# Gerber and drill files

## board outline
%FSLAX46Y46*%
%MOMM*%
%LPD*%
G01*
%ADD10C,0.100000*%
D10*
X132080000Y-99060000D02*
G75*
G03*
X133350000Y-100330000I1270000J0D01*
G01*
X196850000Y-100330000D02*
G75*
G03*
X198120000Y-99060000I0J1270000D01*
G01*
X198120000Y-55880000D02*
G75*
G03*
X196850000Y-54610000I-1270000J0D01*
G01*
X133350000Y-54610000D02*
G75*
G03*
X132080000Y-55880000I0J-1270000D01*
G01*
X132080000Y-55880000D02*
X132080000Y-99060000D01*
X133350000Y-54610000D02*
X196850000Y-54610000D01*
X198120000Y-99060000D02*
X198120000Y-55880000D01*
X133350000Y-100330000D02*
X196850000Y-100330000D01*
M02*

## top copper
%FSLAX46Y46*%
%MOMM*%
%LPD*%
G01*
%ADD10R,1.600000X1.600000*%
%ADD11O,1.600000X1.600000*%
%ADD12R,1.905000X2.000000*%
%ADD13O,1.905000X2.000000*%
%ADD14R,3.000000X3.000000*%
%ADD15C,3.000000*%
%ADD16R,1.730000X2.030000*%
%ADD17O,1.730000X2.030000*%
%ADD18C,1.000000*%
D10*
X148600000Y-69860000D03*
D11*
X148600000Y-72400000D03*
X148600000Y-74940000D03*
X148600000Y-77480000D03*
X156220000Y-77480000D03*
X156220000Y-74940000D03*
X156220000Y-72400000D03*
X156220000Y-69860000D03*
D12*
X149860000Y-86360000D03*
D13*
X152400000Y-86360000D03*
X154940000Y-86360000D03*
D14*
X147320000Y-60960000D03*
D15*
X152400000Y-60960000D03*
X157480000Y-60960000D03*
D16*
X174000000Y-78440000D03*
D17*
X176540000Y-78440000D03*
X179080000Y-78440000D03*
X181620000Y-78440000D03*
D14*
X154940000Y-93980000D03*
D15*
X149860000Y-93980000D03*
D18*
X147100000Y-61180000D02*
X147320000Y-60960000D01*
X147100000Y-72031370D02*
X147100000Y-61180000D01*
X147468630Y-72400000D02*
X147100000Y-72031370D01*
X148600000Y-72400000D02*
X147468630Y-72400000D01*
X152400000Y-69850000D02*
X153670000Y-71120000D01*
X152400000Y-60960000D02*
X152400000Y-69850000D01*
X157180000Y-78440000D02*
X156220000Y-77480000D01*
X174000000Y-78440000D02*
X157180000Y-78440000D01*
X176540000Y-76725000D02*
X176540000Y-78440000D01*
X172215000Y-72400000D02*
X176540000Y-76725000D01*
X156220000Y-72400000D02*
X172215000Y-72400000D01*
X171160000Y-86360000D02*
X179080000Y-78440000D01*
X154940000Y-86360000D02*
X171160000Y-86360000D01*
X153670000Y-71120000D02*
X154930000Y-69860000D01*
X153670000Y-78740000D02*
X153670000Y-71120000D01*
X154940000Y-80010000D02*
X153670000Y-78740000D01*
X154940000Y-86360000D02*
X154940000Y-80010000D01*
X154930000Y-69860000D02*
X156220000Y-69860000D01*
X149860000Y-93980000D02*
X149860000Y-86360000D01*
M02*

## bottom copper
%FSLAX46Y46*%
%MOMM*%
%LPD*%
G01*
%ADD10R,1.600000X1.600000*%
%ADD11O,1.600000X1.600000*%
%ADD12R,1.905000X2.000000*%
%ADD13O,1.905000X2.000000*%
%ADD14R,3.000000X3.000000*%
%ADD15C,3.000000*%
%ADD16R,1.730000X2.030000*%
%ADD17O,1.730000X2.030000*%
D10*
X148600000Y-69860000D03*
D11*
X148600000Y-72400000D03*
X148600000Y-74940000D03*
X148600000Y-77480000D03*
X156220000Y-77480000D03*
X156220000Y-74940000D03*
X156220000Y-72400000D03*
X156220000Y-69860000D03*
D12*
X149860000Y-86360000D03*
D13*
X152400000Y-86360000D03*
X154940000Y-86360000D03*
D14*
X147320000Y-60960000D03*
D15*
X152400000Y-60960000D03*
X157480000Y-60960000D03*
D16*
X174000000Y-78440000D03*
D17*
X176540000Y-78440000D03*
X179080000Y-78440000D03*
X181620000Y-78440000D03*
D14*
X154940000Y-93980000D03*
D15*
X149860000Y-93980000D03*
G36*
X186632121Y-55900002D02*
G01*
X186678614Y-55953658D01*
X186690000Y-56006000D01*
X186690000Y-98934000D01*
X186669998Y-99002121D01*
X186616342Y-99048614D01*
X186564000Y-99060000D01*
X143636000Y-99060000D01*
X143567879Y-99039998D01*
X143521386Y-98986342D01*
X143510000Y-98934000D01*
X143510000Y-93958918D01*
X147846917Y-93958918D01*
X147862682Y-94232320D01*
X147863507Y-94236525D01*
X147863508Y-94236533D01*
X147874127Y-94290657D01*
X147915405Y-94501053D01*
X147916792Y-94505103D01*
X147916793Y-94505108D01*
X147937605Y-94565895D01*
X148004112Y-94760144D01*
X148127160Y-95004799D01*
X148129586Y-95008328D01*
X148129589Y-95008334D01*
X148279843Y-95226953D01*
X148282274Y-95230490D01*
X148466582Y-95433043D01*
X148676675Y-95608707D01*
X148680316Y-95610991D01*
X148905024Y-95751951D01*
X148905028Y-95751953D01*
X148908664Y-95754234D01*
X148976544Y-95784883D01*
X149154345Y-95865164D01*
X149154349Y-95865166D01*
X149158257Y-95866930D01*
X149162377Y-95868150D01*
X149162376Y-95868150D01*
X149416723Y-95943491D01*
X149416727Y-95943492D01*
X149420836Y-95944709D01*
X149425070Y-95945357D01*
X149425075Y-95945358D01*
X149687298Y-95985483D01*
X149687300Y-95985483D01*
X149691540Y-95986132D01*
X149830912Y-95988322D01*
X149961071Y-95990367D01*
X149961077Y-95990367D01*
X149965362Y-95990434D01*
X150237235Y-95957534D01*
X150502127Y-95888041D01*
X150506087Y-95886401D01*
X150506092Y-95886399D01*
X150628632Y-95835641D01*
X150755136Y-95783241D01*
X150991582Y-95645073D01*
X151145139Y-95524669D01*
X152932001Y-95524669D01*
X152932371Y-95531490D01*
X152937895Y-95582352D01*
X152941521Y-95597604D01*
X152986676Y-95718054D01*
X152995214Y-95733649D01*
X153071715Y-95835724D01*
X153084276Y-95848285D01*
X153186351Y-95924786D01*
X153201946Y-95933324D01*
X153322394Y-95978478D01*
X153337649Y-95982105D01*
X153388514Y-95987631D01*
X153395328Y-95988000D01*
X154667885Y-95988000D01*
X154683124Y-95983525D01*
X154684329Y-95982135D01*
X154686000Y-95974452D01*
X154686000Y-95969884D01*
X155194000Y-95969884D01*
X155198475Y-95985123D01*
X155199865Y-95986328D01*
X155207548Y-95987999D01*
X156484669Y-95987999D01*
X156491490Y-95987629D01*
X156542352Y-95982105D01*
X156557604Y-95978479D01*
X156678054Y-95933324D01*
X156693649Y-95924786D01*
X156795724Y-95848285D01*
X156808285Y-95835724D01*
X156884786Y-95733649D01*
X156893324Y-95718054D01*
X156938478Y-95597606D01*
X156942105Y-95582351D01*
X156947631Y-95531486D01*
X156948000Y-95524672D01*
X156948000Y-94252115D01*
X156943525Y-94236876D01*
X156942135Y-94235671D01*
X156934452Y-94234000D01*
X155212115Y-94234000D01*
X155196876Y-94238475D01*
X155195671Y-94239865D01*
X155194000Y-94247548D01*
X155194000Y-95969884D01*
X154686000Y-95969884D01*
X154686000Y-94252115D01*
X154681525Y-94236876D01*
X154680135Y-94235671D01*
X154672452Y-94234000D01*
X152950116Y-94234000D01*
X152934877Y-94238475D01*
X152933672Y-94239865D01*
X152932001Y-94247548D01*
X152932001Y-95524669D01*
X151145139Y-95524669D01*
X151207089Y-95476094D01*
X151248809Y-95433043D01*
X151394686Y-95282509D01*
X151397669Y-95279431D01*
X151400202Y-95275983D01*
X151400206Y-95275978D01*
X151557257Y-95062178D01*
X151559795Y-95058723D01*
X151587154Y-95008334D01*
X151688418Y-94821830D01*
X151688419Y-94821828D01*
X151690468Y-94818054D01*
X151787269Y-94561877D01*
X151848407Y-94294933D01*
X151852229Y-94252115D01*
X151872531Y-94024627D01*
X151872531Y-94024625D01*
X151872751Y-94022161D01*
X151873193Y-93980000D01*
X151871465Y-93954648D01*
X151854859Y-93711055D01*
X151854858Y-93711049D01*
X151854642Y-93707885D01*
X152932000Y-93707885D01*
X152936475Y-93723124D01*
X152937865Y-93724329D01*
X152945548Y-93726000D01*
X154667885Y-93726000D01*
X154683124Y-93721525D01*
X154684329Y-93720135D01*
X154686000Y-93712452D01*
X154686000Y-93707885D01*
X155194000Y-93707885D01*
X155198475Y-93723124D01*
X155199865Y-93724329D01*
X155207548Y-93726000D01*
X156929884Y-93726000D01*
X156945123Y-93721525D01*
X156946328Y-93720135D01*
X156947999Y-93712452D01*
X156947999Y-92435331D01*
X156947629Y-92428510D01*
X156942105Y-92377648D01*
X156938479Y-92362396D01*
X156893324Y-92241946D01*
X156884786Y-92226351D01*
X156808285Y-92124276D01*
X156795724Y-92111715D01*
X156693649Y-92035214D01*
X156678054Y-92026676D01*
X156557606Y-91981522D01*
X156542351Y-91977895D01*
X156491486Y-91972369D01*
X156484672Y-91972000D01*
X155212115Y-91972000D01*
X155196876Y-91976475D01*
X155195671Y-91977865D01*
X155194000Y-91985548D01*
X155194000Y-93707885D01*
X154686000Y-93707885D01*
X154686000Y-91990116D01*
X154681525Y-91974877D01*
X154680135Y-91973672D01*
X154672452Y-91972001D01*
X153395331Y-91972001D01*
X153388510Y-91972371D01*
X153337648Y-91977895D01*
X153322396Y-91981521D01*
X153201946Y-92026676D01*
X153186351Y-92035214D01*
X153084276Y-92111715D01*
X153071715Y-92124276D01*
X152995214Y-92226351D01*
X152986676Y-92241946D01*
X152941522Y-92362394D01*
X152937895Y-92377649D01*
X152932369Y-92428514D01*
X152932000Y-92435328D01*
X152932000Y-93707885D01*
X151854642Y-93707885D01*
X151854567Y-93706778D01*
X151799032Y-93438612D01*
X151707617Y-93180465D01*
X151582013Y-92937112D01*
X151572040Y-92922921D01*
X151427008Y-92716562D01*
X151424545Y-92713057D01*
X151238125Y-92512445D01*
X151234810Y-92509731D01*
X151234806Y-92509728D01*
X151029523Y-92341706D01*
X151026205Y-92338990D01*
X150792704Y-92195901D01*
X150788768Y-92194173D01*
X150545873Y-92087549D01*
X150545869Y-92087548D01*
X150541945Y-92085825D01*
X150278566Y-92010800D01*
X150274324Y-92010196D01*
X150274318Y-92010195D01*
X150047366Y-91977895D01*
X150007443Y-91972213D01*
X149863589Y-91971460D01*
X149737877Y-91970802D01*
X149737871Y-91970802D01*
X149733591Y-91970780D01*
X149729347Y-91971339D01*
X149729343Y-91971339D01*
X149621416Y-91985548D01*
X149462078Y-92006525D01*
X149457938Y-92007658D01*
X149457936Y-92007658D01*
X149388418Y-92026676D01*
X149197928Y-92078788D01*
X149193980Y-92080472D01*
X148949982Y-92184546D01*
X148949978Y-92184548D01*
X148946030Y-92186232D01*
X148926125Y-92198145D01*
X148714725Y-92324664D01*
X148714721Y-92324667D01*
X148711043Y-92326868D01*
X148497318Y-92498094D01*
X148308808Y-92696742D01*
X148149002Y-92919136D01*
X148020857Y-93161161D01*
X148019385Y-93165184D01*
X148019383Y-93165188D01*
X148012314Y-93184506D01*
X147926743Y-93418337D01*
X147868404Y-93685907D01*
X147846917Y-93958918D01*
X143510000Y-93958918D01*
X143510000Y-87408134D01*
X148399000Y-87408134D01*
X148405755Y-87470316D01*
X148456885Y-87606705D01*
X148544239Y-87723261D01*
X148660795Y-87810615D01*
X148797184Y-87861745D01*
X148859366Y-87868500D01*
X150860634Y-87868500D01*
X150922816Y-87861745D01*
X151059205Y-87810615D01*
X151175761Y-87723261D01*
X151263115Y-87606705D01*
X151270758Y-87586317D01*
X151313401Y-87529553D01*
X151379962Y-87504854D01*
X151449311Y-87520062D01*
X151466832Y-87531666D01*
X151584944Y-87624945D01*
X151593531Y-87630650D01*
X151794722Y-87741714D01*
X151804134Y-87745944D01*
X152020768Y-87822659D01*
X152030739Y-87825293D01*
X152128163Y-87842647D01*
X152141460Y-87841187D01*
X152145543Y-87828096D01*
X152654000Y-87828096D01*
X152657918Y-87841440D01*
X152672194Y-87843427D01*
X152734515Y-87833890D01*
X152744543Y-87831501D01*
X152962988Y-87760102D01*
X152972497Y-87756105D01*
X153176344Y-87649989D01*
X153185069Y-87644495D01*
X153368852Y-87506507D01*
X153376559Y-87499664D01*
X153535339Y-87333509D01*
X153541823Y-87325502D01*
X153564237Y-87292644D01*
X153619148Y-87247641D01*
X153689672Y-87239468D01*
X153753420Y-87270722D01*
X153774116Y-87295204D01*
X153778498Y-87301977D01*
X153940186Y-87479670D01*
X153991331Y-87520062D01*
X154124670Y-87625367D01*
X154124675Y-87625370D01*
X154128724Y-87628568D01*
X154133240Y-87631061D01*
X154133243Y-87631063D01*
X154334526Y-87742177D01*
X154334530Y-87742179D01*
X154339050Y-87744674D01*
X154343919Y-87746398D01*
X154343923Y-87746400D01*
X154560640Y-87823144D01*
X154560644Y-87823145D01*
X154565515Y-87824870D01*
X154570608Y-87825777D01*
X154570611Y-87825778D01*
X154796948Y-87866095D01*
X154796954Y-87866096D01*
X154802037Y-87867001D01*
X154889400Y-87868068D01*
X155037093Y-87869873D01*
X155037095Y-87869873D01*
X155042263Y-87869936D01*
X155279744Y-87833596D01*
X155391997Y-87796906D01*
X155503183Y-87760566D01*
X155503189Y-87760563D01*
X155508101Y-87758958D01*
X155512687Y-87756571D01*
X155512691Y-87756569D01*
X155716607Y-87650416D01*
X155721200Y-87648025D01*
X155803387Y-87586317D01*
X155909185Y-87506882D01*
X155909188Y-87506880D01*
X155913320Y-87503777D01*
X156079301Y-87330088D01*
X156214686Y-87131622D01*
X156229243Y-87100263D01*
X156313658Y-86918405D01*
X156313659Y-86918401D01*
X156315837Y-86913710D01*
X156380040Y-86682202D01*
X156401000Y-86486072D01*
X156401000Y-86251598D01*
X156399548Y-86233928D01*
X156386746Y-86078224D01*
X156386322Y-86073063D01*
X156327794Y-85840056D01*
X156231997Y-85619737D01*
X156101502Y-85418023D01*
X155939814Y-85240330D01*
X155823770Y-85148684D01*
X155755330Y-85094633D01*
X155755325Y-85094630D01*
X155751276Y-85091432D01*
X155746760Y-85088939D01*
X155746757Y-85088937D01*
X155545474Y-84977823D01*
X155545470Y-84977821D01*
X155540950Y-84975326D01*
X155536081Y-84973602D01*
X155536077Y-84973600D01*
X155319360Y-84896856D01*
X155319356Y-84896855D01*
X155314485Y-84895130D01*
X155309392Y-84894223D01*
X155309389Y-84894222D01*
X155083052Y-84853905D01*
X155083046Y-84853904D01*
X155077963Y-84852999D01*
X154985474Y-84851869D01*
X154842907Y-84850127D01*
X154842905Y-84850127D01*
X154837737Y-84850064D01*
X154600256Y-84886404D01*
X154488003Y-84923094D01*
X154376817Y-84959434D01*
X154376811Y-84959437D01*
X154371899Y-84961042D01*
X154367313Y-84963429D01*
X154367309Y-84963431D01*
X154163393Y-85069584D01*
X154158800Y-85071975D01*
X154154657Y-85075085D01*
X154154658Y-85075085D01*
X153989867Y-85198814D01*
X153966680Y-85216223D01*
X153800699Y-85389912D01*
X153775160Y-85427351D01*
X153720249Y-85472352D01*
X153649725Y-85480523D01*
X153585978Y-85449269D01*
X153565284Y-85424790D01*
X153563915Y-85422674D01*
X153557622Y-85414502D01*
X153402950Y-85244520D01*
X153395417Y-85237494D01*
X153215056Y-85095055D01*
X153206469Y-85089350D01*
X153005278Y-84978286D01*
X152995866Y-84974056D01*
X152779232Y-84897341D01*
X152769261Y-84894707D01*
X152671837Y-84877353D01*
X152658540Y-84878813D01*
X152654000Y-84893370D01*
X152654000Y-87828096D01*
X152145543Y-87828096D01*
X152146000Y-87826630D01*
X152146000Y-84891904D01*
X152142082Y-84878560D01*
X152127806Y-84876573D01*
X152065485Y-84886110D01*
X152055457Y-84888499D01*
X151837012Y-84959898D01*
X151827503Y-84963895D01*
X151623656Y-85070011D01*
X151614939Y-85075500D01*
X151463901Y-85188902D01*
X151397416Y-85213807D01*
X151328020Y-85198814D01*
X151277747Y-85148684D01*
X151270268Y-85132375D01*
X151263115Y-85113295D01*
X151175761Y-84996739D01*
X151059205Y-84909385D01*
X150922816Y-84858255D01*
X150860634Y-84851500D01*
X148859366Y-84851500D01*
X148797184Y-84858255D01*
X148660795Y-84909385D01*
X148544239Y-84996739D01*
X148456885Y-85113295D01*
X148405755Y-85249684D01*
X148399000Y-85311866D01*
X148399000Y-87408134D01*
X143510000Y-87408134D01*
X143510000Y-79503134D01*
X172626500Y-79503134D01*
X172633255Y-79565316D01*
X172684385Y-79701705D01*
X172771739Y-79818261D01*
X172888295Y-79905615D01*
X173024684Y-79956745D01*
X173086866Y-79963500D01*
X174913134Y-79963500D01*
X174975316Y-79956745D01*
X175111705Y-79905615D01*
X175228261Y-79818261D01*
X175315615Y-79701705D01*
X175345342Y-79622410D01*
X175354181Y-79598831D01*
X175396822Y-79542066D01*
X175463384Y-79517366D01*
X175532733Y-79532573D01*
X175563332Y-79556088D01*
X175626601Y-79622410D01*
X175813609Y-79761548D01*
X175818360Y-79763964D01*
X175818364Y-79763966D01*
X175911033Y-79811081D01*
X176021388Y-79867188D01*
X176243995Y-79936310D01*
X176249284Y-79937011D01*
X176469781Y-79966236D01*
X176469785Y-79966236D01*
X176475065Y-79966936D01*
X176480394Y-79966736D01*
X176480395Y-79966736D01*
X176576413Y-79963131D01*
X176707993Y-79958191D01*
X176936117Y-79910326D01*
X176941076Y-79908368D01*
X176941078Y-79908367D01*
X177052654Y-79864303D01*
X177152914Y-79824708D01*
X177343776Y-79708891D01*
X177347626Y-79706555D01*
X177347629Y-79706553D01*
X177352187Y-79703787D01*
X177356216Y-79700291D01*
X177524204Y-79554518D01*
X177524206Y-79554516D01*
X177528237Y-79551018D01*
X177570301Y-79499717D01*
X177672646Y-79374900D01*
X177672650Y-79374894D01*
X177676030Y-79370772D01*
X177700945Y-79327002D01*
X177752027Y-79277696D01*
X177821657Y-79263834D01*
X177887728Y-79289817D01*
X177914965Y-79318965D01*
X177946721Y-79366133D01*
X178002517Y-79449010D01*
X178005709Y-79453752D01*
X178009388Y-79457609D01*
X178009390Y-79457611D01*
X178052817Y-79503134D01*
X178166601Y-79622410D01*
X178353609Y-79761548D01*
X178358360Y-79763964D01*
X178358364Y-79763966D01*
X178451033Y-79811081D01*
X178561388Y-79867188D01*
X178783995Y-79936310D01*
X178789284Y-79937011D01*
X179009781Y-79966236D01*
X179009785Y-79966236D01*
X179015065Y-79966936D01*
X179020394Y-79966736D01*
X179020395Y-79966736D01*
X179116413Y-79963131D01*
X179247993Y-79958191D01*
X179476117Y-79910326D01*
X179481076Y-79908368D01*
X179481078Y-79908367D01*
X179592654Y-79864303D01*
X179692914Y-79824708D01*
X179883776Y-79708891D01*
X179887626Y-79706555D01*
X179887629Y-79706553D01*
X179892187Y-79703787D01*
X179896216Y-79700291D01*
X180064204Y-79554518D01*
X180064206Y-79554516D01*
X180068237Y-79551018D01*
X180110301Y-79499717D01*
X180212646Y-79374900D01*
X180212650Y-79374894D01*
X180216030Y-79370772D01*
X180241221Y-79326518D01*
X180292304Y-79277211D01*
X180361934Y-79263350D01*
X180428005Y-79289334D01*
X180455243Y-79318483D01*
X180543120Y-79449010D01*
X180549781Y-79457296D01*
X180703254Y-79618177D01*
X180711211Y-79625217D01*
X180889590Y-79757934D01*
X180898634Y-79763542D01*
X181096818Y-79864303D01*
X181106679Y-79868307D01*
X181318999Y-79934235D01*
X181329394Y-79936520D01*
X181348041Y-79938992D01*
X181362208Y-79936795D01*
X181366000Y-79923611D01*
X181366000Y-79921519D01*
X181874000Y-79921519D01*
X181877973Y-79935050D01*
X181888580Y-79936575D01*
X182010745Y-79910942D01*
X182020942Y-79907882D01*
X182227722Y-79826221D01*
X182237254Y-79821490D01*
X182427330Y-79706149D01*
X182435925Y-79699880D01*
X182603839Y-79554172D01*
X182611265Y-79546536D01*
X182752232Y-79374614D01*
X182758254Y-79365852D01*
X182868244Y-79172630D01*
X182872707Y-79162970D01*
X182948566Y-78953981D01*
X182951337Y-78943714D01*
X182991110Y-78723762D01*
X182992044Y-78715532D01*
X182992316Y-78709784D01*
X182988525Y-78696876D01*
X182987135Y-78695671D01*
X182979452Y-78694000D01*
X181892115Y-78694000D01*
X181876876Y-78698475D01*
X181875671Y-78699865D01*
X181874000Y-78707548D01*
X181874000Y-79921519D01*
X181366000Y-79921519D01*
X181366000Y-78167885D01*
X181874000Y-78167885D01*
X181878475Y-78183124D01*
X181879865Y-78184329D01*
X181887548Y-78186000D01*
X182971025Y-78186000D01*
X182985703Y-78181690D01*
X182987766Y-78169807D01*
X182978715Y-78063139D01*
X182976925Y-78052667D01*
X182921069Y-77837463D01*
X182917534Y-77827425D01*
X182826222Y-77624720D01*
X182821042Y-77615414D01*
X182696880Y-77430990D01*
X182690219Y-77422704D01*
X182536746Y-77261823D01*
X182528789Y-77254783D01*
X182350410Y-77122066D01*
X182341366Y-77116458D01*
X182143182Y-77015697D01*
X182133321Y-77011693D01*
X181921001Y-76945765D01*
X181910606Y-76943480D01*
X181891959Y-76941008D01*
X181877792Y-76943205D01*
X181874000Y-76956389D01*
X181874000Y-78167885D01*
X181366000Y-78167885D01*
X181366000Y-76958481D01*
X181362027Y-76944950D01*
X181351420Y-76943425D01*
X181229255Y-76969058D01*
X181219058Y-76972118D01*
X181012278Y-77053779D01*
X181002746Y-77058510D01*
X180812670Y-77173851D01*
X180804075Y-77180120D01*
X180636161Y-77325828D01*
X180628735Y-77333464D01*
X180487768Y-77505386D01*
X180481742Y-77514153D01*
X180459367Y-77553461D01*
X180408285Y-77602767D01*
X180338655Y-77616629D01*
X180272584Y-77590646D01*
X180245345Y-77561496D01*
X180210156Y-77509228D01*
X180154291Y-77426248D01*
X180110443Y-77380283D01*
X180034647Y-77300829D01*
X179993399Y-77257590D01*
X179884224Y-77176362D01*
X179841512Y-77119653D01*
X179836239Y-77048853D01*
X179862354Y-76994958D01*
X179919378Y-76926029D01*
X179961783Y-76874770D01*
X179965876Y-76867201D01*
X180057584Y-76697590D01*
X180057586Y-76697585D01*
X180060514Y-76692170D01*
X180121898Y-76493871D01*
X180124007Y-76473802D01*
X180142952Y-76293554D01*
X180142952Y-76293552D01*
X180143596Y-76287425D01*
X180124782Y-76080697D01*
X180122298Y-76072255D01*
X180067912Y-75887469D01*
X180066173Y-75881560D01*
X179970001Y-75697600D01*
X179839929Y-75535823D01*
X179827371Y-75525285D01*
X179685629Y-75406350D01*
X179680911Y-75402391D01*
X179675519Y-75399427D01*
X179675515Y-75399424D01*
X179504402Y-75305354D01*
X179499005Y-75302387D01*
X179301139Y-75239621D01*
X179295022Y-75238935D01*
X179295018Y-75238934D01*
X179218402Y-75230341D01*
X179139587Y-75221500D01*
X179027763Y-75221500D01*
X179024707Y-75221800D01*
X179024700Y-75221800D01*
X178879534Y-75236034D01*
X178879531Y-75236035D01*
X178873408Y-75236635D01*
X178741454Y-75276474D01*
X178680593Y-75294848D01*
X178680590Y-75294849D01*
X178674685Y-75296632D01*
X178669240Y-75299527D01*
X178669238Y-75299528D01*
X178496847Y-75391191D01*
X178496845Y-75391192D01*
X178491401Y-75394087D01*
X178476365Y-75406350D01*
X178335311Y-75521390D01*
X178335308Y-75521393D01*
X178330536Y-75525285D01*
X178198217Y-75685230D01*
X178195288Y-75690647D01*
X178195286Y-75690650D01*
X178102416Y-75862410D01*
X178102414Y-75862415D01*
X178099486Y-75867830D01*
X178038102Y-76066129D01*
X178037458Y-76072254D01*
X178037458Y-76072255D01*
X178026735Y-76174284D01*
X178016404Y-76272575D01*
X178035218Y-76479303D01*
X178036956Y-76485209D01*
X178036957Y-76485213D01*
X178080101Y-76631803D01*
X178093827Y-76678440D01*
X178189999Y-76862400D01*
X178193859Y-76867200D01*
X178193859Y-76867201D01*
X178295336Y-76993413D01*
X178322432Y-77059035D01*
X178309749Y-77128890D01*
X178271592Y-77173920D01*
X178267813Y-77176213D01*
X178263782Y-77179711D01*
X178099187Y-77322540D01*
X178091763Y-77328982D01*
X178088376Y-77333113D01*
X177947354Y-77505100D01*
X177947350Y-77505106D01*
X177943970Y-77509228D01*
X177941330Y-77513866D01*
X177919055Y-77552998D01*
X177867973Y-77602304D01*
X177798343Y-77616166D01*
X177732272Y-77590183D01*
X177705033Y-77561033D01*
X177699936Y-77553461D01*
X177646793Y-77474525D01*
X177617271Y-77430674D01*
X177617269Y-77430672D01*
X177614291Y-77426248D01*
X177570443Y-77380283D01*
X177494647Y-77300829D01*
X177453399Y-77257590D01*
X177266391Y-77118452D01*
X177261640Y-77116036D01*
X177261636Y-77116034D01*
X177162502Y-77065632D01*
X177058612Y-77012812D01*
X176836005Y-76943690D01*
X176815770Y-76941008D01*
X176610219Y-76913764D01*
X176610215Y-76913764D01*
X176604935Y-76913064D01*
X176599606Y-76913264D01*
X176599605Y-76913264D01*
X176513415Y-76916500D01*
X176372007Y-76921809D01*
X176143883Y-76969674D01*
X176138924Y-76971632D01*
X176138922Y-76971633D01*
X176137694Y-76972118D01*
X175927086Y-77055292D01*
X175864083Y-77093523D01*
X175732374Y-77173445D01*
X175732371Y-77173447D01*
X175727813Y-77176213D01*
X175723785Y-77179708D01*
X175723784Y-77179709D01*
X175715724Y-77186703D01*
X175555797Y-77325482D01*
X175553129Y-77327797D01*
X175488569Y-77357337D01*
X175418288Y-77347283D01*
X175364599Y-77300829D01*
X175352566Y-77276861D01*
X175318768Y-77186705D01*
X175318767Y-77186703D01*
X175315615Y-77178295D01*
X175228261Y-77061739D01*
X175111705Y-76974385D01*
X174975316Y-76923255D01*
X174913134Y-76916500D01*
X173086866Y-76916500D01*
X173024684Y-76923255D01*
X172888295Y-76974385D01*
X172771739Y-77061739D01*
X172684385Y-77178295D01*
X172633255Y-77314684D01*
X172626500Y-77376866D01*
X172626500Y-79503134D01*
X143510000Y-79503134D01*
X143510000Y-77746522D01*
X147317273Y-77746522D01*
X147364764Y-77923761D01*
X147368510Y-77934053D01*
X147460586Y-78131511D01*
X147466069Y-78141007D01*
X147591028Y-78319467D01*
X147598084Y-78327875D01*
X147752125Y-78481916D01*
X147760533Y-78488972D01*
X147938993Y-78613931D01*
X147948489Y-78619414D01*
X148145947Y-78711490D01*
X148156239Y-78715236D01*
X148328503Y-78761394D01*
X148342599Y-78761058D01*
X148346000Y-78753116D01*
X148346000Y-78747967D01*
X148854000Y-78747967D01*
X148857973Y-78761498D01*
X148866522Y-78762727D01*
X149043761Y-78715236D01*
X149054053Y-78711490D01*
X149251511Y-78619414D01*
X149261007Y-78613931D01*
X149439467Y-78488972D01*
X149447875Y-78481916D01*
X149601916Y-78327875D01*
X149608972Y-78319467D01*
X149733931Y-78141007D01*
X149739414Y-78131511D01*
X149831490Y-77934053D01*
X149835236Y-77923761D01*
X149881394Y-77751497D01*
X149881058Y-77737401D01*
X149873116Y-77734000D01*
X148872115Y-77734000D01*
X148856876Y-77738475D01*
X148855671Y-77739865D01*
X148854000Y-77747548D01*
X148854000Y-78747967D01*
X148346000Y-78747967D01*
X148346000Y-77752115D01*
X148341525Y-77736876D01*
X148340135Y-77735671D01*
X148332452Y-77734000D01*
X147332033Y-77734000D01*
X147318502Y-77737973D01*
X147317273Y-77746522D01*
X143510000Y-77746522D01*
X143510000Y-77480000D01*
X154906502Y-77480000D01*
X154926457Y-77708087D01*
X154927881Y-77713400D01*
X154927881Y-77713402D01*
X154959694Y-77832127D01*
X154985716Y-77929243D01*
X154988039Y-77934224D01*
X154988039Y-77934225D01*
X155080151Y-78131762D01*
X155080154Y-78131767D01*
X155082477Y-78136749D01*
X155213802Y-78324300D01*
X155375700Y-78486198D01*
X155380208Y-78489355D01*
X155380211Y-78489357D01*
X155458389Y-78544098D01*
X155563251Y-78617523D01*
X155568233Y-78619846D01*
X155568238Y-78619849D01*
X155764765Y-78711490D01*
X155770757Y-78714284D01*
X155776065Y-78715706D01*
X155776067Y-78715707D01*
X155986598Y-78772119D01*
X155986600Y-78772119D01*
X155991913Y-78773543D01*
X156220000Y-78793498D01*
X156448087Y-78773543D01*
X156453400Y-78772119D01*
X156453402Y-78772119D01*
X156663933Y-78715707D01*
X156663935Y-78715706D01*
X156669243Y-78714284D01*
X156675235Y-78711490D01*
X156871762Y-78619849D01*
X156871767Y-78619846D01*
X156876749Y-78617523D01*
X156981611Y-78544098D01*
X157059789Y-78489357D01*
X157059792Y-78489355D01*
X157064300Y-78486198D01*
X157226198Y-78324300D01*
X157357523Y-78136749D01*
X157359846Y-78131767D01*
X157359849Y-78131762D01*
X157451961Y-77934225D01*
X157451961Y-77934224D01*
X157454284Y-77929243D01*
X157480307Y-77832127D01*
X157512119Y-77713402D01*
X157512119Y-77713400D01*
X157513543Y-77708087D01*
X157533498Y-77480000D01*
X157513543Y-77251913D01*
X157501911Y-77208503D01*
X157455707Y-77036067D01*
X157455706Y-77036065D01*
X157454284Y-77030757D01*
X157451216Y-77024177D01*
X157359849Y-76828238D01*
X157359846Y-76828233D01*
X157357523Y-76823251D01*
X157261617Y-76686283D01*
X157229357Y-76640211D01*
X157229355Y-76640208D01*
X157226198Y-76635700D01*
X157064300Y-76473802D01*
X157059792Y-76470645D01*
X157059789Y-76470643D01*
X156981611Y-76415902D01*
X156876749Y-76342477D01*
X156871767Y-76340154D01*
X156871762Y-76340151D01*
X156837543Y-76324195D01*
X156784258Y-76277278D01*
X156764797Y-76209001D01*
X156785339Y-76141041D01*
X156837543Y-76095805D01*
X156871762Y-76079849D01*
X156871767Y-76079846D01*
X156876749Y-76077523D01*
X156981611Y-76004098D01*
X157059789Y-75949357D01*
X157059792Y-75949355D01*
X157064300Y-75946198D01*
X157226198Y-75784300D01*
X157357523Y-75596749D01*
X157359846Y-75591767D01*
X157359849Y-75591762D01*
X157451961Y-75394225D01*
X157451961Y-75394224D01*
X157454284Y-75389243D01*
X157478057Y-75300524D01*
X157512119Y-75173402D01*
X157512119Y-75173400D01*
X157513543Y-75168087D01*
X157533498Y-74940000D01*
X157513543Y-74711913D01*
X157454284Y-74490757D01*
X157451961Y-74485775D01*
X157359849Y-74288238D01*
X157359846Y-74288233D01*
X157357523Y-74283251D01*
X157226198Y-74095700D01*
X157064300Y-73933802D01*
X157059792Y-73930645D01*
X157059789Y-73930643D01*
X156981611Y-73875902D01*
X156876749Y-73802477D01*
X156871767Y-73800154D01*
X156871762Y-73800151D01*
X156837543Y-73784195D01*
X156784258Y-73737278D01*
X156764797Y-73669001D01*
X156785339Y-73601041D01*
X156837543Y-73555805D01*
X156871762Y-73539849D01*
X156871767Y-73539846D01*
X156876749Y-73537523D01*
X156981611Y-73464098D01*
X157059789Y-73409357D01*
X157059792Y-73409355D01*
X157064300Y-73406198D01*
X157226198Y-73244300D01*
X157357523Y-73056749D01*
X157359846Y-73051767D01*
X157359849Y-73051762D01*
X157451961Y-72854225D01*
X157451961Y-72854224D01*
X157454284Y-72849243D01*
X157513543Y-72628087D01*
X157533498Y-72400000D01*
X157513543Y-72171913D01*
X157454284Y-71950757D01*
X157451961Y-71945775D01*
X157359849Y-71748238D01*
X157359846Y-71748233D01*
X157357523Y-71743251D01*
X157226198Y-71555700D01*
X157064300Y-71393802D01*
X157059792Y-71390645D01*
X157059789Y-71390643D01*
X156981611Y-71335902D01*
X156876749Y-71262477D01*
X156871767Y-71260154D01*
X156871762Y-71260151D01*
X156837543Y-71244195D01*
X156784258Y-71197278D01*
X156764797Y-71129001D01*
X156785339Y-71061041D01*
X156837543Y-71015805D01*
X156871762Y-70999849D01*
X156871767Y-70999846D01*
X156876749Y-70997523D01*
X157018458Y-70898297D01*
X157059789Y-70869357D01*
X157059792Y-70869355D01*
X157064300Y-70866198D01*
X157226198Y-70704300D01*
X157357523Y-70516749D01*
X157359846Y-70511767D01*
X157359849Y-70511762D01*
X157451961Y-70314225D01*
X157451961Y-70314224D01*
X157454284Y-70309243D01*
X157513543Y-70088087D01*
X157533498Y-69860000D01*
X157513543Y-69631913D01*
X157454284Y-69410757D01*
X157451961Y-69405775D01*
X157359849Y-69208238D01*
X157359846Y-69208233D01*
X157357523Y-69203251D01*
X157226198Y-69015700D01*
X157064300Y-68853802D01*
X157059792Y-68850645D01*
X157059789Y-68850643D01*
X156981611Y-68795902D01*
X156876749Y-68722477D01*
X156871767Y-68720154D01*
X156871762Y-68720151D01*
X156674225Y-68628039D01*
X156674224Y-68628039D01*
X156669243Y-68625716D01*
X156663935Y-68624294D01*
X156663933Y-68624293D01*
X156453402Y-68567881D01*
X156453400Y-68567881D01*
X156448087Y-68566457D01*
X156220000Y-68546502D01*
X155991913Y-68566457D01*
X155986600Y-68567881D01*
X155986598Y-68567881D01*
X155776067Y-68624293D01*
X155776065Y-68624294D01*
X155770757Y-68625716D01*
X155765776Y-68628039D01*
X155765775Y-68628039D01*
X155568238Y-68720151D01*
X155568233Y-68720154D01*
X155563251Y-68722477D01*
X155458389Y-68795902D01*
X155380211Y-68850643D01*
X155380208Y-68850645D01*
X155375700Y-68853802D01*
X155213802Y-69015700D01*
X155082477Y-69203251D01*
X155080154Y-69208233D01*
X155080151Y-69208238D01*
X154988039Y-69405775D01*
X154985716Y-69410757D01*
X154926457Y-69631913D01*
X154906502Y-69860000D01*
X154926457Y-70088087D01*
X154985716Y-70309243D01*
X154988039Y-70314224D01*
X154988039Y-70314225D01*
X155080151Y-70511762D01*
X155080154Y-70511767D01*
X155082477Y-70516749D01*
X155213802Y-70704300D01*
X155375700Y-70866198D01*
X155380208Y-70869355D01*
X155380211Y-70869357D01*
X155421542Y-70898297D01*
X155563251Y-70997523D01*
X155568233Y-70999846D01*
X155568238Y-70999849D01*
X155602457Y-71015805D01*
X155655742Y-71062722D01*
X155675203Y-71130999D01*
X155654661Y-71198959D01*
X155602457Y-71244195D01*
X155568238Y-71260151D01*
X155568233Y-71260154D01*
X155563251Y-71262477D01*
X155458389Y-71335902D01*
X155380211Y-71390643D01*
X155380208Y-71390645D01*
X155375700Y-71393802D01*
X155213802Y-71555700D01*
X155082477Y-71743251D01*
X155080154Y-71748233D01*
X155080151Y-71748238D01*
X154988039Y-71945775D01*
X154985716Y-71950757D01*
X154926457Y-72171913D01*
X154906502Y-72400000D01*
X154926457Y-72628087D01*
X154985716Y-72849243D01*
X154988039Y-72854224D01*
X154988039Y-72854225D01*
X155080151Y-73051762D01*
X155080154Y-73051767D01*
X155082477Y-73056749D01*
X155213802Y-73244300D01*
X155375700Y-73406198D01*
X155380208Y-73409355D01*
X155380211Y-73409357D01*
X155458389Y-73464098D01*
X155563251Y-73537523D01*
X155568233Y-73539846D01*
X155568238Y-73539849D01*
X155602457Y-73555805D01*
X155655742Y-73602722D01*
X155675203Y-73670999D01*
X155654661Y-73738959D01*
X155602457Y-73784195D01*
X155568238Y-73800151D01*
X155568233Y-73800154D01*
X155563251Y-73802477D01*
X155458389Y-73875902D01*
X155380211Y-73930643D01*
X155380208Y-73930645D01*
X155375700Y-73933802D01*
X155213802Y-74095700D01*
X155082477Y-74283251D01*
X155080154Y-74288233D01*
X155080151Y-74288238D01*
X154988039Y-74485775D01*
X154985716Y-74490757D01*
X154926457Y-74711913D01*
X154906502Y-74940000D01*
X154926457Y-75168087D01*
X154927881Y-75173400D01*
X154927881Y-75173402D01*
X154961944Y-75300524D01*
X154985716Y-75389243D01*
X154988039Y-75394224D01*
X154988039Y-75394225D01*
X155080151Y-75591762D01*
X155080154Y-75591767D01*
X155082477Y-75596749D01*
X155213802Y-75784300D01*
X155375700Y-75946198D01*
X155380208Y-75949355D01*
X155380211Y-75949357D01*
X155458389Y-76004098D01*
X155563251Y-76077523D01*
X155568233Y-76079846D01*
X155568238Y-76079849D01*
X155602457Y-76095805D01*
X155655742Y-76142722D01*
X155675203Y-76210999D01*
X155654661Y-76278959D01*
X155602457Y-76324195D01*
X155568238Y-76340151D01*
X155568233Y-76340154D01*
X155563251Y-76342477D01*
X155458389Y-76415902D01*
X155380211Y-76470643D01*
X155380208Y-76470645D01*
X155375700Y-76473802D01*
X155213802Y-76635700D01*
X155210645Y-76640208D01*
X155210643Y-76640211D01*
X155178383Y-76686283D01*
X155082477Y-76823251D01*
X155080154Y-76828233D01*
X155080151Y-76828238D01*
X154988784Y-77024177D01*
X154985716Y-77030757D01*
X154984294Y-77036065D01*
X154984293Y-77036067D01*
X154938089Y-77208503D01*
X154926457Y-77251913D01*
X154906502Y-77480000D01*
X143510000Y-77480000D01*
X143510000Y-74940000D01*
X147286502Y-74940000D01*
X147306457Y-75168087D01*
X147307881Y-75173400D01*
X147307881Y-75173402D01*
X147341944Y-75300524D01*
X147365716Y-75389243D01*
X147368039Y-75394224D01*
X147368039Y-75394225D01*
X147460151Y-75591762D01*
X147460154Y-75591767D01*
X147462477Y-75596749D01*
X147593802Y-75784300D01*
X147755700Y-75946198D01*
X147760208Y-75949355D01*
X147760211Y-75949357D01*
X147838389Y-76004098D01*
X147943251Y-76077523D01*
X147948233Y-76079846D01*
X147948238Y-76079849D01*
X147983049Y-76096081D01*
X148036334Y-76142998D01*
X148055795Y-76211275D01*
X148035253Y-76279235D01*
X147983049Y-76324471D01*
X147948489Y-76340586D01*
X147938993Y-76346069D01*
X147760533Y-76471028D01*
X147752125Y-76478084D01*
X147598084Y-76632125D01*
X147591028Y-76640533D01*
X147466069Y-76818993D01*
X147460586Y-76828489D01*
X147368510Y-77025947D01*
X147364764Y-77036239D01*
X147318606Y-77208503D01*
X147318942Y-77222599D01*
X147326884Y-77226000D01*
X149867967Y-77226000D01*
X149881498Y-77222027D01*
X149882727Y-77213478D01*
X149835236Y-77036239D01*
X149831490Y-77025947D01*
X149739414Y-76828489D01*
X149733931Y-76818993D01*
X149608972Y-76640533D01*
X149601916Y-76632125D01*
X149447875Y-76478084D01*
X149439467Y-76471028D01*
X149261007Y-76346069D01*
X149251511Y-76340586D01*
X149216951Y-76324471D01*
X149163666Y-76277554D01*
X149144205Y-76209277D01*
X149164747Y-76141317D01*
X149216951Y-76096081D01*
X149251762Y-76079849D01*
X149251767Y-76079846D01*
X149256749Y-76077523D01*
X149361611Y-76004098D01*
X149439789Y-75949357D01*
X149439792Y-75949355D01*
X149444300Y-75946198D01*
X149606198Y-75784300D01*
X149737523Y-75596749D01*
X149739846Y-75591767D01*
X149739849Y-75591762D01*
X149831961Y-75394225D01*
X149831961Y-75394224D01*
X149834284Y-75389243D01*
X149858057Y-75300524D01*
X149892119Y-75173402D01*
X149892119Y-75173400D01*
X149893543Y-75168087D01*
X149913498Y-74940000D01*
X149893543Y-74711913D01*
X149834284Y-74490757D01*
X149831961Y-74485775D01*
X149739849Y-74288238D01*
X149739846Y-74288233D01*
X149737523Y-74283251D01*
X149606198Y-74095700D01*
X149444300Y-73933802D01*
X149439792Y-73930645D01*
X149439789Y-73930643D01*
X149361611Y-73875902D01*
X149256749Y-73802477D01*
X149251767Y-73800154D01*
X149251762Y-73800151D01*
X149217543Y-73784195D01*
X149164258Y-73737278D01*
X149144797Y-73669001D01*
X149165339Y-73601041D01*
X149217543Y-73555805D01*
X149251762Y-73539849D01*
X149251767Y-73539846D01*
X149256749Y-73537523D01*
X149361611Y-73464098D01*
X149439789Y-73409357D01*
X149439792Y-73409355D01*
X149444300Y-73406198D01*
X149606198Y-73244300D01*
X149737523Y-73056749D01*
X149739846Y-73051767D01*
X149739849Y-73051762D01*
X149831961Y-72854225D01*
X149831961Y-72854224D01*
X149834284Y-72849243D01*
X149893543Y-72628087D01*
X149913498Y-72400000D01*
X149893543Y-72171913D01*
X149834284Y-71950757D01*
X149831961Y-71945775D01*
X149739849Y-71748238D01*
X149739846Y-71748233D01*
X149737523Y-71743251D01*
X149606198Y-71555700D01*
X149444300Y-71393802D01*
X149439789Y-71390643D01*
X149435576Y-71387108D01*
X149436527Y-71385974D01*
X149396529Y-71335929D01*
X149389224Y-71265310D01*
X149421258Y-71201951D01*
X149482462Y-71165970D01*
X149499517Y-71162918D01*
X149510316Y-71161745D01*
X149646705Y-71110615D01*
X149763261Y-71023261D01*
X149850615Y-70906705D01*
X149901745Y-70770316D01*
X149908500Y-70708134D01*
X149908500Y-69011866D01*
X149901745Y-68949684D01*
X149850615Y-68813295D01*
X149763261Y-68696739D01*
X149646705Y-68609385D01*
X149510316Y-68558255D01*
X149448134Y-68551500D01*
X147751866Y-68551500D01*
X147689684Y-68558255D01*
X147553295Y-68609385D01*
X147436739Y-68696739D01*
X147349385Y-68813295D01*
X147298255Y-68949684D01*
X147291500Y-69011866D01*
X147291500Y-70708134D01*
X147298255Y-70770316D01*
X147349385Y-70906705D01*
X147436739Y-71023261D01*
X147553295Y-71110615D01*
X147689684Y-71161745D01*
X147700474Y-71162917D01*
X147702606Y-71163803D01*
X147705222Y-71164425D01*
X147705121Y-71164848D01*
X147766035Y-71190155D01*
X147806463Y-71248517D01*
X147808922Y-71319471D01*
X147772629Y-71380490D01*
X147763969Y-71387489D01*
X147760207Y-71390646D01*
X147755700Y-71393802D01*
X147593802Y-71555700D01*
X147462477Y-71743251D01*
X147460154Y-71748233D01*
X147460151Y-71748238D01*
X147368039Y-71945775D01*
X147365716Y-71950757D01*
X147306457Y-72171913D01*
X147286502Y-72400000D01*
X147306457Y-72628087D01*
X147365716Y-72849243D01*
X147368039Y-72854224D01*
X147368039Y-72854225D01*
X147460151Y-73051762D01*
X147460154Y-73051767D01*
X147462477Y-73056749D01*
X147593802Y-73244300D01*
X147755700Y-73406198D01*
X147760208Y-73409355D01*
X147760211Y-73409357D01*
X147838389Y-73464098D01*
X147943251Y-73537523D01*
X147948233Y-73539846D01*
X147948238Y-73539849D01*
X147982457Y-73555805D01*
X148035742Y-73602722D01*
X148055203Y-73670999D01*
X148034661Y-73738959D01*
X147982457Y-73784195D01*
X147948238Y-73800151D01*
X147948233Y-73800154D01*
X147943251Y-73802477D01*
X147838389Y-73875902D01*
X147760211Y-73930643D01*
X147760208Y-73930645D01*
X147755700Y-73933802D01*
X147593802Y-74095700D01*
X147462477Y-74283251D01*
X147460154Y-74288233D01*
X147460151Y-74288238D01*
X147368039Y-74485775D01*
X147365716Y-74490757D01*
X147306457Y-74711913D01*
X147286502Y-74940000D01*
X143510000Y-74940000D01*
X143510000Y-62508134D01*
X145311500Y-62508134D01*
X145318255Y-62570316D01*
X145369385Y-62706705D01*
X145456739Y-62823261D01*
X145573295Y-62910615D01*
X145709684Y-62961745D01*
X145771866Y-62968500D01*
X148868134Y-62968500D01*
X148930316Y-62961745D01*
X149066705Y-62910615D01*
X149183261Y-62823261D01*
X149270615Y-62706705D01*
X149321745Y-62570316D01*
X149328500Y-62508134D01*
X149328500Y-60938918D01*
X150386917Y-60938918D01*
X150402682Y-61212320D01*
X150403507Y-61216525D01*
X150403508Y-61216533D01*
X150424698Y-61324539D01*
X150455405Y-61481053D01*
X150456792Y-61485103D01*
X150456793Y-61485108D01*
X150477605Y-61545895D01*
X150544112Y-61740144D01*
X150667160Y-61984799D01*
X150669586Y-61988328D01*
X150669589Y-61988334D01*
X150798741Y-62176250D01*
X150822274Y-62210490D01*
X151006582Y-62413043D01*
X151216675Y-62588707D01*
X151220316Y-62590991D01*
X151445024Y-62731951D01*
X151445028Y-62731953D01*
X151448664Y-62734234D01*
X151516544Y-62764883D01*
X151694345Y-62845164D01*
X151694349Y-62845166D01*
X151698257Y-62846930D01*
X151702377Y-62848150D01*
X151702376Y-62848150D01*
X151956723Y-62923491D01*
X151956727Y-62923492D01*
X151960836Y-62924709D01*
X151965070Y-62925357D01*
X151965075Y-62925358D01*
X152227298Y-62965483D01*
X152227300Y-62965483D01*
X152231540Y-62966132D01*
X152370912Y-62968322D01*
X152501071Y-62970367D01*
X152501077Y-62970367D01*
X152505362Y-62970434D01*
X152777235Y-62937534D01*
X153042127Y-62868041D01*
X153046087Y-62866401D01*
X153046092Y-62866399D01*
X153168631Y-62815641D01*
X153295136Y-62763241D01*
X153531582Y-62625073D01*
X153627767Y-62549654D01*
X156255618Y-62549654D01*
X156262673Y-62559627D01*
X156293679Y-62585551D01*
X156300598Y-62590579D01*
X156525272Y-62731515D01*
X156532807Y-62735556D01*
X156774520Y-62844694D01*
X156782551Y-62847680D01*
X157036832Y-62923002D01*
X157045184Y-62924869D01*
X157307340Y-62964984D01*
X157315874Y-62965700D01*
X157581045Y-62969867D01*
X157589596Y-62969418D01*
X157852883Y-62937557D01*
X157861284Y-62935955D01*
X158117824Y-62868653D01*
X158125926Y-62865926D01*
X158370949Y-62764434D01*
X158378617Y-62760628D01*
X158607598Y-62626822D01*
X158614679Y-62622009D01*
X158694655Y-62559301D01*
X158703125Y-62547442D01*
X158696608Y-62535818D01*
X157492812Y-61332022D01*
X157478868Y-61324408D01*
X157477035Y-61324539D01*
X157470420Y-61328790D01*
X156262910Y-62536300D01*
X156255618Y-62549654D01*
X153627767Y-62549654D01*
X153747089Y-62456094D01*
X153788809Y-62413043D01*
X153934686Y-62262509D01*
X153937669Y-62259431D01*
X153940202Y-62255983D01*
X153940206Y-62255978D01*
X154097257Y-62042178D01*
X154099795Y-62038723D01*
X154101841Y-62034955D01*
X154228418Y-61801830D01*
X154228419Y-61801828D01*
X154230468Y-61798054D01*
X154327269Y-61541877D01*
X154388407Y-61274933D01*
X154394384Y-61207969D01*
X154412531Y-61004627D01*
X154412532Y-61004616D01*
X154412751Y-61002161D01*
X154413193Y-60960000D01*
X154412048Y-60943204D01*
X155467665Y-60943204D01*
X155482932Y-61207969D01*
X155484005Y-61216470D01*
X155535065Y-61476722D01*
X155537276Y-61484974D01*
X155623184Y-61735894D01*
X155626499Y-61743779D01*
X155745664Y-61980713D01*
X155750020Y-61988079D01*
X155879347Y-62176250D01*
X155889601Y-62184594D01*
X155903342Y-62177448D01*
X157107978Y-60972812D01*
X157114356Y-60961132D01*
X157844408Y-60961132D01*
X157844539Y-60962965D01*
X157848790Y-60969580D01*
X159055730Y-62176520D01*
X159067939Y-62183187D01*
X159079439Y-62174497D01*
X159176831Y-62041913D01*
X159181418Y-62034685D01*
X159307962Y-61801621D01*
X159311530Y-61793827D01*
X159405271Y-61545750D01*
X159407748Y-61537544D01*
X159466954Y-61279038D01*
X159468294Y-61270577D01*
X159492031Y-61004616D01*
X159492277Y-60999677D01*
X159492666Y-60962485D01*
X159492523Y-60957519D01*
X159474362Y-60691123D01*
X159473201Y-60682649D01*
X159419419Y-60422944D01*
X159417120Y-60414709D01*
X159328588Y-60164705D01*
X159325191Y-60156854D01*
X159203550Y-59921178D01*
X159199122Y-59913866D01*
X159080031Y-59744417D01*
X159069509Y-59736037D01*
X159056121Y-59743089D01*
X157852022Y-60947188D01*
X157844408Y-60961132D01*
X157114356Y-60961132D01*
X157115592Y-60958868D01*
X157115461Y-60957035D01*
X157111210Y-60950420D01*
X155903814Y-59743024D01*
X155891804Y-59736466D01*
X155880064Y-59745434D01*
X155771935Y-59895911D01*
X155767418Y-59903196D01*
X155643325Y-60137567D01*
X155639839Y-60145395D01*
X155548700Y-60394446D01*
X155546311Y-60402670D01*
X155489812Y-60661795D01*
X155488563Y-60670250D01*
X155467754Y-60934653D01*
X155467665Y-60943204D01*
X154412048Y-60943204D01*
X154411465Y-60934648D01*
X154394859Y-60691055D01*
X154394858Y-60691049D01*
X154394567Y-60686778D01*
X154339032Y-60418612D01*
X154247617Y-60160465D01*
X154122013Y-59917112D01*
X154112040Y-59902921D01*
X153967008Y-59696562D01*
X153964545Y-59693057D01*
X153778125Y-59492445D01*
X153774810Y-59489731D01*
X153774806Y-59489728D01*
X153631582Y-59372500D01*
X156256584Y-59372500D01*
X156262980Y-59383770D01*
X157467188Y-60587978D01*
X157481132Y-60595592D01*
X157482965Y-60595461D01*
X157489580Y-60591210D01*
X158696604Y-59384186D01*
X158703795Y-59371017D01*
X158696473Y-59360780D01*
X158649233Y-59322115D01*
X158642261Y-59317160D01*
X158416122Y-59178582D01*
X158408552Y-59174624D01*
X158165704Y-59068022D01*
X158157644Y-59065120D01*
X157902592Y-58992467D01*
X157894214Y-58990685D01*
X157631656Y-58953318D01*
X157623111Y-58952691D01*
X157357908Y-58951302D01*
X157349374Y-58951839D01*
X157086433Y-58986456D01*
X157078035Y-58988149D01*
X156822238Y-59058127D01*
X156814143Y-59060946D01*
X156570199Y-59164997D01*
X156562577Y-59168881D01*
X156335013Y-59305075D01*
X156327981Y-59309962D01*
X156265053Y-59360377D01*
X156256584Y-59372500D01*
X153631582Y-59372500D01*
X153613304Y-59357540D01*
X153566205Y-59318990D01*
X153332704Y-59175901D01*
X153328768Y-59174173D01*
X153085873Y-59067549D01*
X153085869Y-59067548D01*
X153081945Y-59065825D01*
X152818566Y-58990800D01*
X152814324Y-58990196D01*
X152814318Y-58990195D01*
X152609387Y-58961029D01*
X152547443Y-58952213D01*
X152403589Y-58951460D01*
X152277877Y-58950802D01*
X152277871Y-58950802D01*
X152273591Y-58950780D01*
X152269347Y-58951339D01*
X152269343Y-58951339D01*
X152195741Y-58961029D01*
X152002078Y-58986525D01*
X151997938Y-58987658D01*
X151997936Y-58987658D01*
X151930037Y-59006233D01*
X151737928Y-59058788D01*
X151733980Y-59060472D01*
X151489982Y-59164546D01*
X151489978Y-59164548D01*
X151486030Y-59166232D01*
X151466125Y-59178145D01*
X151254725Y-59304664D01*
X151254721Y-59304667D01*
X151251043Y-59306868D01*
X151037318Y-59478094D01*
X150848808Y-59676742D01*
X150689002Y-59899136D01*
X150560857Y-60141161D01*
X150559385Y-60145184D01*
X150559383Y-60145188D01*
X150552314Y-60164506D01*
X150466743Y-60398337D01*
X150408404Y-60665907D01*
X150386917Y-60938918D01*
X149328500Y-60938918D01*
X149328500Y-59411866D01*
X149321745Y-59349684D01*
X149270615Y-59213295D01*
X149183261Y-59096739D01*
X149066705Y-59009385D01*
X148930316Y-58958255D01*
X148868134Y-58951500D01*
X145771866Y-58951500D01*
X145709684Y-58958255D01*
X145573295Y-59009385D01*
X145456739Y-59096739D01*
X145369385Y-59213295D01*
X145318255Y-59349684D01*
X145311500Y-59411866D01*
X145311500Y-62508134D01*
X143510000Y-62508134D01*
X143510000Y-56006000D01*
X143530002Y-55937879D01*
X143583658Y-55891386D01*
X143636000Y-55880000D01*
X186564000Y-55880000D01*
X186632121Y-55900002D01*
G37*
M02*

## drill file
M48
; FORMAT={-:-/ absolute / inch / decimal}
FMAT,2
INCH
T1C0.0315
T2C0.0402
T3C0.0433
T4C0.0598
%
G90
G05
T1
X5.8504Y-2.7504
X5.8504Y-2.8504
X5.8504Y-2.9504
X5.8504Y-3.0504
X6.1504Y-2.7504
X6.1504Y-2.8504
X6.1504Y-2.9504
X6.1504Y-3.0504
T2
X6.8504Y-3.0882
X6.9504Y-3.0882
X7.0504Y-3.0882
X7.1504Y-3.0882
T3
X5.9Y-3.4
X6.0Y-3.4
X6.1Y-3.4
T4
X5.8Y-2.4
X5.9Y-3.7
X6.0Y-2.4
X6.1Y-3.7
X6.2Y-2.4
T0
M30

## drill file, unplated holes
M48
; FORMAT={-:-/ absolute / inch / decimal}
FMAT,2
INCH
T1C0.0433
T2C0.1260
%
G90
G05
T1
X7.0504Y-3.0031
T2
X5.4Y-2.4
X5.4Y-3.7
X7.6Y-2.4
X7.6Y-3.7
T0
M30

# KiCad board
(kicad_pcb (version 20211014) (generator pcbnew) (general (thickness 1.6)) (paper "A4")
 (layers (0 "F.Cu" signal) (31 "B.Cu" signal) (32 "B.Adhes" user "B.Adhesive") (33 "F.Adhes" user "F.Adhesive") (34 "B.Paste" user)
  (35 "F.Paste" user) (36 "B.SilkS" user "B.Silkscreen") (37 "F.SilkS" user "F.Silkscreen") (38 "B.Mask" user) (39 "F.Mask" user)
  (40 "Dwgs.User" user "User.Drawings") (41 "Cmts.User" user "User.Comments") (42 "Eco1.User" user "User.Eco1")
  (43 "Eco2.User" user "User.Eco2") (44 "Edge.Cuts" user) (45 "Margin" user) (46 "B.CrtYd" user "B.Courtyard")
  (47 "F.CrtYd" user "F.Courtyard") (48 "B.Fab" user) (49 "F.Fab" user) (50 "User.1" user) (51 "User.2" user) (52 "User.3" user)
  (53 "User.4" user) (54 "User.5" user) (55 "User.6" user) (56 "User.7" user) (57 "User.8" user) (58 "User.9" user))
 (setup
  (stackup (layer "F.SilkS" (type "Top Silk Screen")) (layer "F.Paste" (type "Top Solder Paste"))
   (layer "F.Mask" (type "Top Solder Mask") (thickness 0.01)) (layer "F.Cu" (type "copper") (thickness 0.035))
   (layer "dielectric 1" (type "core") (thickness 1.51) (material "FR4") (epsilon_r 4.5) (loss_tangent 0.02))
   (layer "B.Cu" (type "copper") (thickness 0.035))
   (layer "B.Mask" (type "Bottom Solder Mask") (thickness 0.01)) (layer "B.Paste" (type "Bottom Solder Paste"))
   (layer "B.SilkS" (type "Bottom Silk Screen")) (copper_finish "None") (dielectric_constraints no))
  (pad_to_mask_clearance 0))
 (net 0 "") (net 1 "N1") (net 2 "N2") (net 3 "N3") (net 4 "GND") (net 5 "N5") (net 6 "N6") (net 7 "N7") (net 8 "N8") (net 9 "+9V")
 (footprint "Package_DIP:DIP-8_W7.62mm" (layer "F.Cu") (at 148.6 69.86)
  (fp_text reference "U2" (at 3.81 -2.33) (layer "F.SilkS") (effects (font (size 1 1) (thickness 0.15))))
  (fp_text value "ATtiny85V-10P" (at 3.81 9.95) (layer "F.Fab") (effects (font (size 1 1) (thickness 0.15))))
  (pad "1" thru_hole rect (at 0 0) (size 1.6 1.6) (drill 0.8) (layers *.Cu *.Mask) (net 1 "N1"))
  (pad "2" thru_hole oval (at 0 2.54) (size 1.6 1.6) (drill 0.8) (layers *.Cu *.Mask) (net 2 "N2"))
  (pad "3" thru_hole oval (at 0 5.08) (size 1.6 1.6) (drill 0.8) (layers *.Cu *.Mask) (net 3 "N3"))
  (pad "4" thru_hole oval (at 0 7.62) (size 1.6 1.6) (drill 0.8) (layers *.Cu *.Mask) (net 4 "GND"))
  (pad "5" thru_hole oval (at 7.62 7.62) (size 1.6 1.6) (drill 0.8) (layers *.Cu *.Mask) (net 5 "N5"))
  (pad "6" thru_hole oval (at 7.62 5.08) (size 1.6 1.6) (drill 0.8) (layers *.Cu *.Mask) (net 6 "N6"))
  (pad "7" thru_hole oval (at 7.62 2.54) (size 1.6 1.6) (drill 0.8) (layers *.Cu *.Mask) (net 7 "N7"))
  (pad "8" thru_hole oval (at 7.62 0) (size 1.6 1.6) (drill 0.8) (layers *.Cu *.Mask) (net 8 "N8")))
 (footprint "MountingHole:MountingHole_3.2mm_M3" (layer "F.Cu") (at 137.16 93.98)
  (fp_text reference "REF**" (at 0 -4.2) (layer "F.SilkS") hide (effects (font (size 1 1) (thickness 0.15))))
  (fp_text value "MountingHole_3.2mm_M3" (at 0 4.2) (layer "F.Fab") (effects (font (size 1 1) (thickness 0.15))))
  (pad "" np_thru_hole circle (at 0 0) (size 3.2 3.2) (drill 3.2) (layers *.Cu *.Mask)))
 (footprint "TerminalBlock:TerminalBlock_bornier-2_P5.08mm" (layer "F.Cu") (at 154.94 93.98 180)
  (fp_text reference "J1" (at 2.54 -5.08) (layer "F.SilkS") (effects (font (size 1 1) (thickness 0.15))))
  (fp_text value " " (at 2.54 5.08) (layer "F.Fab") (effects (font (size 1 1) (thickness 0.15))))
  (pad "1" thru_hole rect (at 0 0 180) (size 3 3) (drill 1.52) (layers *.Cu *.Mask) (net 4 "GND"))
  (pad "2" thru_hole circle (at 5.08 0 180) (size 3 3) (drill 1.52) (layers *.Cu *.Mask) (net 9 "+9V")))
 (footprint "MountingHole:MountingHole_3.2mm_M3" (layer "F.Cu") (at 193.04 93.98)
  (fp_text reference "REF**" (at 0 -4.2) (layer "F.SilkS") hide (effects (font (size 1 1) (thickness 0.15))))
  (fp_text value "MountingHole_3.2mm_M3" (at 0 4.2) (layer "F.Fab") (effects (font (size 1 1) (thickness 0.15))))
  (pad "" np_thru_hole circle (at 0 0) (size 3.2 3.2) (drill 3.2) (layers F&B.Cu *.Mask)))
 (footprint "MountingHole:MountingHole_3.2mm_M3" (layer "F.Cu") (at 137.16 60.96)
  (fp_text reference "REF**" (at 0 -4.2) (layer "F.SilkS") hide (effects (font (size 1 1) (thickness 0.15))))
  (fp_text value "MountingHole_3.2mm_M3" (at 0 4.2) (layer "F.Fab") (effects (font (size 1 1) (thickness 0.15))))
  (pad "" np_thru_hole circle (at 0 0) (size 3.2 3.2) (drill 3.2) (layers F&B.Cu *.Mask)))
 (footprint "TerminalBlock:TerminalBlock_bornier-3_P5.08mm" (layer "F.Cu") (at 147.32 60.96)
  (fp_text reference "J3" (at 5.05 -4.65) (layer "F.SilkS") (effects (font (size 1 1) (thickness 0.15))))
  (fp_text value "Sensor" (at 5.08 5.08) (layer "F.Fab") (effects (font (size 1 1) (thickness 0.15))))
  (pad "1" thru_hole rect (at 0 0) (size 3 3) (drill 1.52) (layers *.Cu *.Mask) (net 2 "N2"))
  (pad "2" thru_hole circle (at 5.08 0) (size 3 3) (drill 1.52) (layers *.Cu *.Mask) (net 8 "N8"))
  (pad "3" thru_hole circle (at 10.16 0) (size 3 3) (drill 1.52) (layers *.Cu *.Mask) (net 4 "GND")))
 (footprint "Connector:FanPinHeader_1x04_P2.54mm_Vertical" (layer "F.Cu") (at 174 78.44)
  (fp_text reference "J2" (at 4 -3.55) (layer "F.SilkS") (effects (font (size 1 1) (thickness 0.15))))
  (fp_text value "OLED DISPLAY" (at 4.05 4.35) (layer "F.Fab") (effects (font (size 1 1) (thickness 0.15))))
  (pad "" np_thru_hole circle (at 5.08 -2.16 90) (size 1.1 1.1) (drill 1.1) (layers *.Cu *.Mask))
  (pad "1" thru_hole rect (at 0 0 90) (size 2.03 1.73) (drill 1.02) (layers *.Cu *.Mask) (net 5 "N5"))
  (pad "2" thru_hole oval (at 2.54 0 90) (size 2.03 1.73) (drill 1.02) (layers *.Cu *.Mask) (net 7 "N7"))
  (pad "3" thru_hole oval (at 5.08 0 90) (size 2.03 1.73) (drill 1.02) (layers *.Cu *.Mask) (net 8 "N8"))
  (pad "4" thru_hole oval (at 7.62 0 90) (size 2.03 1.73) (drill 1.02) (layers *.Cu *.Mask) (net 4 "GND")))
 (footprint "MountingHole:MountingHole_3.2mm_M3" (layer "F.Cu") (at 193.04 60.96)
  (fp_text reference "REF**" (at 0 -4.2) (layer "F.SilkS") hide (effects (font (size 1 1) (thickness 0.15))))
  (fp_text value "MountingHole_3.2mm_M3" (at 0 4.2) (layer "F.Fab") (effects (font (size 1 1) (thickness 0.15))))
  (pad "" np_thru_hole circle (at 0 0) (size 3.2 3.2) (drill 3.2) (layers F&B.Cu *.Mask)))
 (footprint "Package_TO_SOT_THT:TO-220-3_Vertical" (layer "F.Cu") (at 149.86 86.36)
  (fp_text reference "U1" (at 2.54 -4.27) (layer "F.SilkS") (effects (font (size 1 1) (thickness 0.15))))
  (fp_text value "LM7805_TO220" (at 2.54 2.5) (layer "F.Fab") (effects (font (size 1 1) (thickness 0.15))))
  (pad "1" thru_hole rect (at 0 0) (size 1.905 2) (drill 1.1) (layers *.Cu *.Mask) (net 9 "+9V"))
  (pad "2" thru_hole oval (at 2.54 0) (size 1.905 2) (drill 1.1) (layers *.Cu *.Mask) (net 4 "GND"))
  (pad "3" thru_hole oval (at 5.08 0) (size 1.905 2) (drill 1.1) (layers *.Cu *.Mask) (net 8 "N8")))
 (gr_line (start 132.08 55.88) (end 132.08 99.06) (layer "Edge.Cuts") (width 0.1))
 (gr_arc (start 133.35 100.33) (mid 132.451974 99.958026) (end 132.08 99.06) (layer "Edge.Cuts") (width 0.1))
 (gr_line (start 133.35 54.61) (end 196.85 54.61) (layer "Edge.Cuts") (width 0.1))
 (gr_line (start 133.35 100.33) (end 196.85 100.33) (layer "Edge.Cuts") (width 0.1))
 (gr_arc (start 132.08 55.88) (mid 132.451974 54.981974) (end 133.35 54.61) (layer "Edge.Cuts") (width 0.1))
 (gr_arc (start 198.12 99.06) (mid 197.748026 99.958026) (end 196.85 100.33) (layer "Edge.Cuts") (width 0.1))
 (gr_arc (start 196.85 54.61) (mid 197.748026 54.981974) (end 198.12 55.88) (layer "Edge.Cuts") (width 0.1))
 (gr_line (start 198.12 99.06) (end 198.12 55.88) (layer "Edge.Cuts") (width 0.1))
 (segment (start 149.86 93.98) (end 149.86 86.36) (width 1) (layer "F.Cu") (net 9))
 (segment (start 157.18 78.44) (end 156.22 77.48) (width 1) (layer "F.Cu") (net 5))
 (segment (start 174 78.44) (end 157.18 78.44) (width 1) (layer "F.Cu") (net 5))
 (segment (start 172.215 72.4) (end 176.54 76.725) (width 1) (layer "F.Cu") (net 7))
 (segment (start 176.54 76.725) (end 176.54 78.44) (width 1) (layer "F.Cu") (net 7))
 (segment (start 156.22 72.4) (end 172.215 72.4) (width 1) (layer "F.Cu") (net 7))
 (segment (start 152.4 60.96) (end 152.4 69.85) (width 1) (layer "F.Cu") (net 8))
 (segment (start 153.67 71.12) (end 154.93 69.86) (width 1) (layer "F.Cu") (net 8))
 (segment (start 152.4 69.85) (end 153.67 71.12) (width 1) (layer "F.Cu") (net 8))
 (segment (start 154.94 80.01) (end 153.67 78.74) (width 1) (layer "F.Cu") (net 8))
 (segment (start 153.67 78.74) (end 153.67 71.12) (width 1) (layer "F.Cu") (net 8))
 (segment (start 154.94 86.36) (end 171.16 86.36) (width 1) (layer "F.Cu") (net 8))
 (segment (start 171.16 86.36) (end 179.08 78.44) (width 1) (layer "F.Cu") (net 8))
 (segment (start 154.94 86.36) (end 154.94 80.01) (width 1) (layer "F.Cu") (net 8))
 (segment (start 154.93 69.86) (end 156.22 69.86) (width 1) (layer "F.Cu") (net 8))
 (segment (start 147.1 61.18) (end 147.32 60.96) (width 1) (layer "F.Cu") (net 2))
 (segment (start 148.6 72.4) (end 147.46863 72.4) (width 1) (layer "F.Cu") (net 2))
 (segment (start 147.46863 72.4) (end 147.1 72.03137) (width 1) (layer "F.Cu") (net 2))
 (segment (start 147.1 72.03137) (end 147.1 61.18) (width 1) (layer "F.Cu") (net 2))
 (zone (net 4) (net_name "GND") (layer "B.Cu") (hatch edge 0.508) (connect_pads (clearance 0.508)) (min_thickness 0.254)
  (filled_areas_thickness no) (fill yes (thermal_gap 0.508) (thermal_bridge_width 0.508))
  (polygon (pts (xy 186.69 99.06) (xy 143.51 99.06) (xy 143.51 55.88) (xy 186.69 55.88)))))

